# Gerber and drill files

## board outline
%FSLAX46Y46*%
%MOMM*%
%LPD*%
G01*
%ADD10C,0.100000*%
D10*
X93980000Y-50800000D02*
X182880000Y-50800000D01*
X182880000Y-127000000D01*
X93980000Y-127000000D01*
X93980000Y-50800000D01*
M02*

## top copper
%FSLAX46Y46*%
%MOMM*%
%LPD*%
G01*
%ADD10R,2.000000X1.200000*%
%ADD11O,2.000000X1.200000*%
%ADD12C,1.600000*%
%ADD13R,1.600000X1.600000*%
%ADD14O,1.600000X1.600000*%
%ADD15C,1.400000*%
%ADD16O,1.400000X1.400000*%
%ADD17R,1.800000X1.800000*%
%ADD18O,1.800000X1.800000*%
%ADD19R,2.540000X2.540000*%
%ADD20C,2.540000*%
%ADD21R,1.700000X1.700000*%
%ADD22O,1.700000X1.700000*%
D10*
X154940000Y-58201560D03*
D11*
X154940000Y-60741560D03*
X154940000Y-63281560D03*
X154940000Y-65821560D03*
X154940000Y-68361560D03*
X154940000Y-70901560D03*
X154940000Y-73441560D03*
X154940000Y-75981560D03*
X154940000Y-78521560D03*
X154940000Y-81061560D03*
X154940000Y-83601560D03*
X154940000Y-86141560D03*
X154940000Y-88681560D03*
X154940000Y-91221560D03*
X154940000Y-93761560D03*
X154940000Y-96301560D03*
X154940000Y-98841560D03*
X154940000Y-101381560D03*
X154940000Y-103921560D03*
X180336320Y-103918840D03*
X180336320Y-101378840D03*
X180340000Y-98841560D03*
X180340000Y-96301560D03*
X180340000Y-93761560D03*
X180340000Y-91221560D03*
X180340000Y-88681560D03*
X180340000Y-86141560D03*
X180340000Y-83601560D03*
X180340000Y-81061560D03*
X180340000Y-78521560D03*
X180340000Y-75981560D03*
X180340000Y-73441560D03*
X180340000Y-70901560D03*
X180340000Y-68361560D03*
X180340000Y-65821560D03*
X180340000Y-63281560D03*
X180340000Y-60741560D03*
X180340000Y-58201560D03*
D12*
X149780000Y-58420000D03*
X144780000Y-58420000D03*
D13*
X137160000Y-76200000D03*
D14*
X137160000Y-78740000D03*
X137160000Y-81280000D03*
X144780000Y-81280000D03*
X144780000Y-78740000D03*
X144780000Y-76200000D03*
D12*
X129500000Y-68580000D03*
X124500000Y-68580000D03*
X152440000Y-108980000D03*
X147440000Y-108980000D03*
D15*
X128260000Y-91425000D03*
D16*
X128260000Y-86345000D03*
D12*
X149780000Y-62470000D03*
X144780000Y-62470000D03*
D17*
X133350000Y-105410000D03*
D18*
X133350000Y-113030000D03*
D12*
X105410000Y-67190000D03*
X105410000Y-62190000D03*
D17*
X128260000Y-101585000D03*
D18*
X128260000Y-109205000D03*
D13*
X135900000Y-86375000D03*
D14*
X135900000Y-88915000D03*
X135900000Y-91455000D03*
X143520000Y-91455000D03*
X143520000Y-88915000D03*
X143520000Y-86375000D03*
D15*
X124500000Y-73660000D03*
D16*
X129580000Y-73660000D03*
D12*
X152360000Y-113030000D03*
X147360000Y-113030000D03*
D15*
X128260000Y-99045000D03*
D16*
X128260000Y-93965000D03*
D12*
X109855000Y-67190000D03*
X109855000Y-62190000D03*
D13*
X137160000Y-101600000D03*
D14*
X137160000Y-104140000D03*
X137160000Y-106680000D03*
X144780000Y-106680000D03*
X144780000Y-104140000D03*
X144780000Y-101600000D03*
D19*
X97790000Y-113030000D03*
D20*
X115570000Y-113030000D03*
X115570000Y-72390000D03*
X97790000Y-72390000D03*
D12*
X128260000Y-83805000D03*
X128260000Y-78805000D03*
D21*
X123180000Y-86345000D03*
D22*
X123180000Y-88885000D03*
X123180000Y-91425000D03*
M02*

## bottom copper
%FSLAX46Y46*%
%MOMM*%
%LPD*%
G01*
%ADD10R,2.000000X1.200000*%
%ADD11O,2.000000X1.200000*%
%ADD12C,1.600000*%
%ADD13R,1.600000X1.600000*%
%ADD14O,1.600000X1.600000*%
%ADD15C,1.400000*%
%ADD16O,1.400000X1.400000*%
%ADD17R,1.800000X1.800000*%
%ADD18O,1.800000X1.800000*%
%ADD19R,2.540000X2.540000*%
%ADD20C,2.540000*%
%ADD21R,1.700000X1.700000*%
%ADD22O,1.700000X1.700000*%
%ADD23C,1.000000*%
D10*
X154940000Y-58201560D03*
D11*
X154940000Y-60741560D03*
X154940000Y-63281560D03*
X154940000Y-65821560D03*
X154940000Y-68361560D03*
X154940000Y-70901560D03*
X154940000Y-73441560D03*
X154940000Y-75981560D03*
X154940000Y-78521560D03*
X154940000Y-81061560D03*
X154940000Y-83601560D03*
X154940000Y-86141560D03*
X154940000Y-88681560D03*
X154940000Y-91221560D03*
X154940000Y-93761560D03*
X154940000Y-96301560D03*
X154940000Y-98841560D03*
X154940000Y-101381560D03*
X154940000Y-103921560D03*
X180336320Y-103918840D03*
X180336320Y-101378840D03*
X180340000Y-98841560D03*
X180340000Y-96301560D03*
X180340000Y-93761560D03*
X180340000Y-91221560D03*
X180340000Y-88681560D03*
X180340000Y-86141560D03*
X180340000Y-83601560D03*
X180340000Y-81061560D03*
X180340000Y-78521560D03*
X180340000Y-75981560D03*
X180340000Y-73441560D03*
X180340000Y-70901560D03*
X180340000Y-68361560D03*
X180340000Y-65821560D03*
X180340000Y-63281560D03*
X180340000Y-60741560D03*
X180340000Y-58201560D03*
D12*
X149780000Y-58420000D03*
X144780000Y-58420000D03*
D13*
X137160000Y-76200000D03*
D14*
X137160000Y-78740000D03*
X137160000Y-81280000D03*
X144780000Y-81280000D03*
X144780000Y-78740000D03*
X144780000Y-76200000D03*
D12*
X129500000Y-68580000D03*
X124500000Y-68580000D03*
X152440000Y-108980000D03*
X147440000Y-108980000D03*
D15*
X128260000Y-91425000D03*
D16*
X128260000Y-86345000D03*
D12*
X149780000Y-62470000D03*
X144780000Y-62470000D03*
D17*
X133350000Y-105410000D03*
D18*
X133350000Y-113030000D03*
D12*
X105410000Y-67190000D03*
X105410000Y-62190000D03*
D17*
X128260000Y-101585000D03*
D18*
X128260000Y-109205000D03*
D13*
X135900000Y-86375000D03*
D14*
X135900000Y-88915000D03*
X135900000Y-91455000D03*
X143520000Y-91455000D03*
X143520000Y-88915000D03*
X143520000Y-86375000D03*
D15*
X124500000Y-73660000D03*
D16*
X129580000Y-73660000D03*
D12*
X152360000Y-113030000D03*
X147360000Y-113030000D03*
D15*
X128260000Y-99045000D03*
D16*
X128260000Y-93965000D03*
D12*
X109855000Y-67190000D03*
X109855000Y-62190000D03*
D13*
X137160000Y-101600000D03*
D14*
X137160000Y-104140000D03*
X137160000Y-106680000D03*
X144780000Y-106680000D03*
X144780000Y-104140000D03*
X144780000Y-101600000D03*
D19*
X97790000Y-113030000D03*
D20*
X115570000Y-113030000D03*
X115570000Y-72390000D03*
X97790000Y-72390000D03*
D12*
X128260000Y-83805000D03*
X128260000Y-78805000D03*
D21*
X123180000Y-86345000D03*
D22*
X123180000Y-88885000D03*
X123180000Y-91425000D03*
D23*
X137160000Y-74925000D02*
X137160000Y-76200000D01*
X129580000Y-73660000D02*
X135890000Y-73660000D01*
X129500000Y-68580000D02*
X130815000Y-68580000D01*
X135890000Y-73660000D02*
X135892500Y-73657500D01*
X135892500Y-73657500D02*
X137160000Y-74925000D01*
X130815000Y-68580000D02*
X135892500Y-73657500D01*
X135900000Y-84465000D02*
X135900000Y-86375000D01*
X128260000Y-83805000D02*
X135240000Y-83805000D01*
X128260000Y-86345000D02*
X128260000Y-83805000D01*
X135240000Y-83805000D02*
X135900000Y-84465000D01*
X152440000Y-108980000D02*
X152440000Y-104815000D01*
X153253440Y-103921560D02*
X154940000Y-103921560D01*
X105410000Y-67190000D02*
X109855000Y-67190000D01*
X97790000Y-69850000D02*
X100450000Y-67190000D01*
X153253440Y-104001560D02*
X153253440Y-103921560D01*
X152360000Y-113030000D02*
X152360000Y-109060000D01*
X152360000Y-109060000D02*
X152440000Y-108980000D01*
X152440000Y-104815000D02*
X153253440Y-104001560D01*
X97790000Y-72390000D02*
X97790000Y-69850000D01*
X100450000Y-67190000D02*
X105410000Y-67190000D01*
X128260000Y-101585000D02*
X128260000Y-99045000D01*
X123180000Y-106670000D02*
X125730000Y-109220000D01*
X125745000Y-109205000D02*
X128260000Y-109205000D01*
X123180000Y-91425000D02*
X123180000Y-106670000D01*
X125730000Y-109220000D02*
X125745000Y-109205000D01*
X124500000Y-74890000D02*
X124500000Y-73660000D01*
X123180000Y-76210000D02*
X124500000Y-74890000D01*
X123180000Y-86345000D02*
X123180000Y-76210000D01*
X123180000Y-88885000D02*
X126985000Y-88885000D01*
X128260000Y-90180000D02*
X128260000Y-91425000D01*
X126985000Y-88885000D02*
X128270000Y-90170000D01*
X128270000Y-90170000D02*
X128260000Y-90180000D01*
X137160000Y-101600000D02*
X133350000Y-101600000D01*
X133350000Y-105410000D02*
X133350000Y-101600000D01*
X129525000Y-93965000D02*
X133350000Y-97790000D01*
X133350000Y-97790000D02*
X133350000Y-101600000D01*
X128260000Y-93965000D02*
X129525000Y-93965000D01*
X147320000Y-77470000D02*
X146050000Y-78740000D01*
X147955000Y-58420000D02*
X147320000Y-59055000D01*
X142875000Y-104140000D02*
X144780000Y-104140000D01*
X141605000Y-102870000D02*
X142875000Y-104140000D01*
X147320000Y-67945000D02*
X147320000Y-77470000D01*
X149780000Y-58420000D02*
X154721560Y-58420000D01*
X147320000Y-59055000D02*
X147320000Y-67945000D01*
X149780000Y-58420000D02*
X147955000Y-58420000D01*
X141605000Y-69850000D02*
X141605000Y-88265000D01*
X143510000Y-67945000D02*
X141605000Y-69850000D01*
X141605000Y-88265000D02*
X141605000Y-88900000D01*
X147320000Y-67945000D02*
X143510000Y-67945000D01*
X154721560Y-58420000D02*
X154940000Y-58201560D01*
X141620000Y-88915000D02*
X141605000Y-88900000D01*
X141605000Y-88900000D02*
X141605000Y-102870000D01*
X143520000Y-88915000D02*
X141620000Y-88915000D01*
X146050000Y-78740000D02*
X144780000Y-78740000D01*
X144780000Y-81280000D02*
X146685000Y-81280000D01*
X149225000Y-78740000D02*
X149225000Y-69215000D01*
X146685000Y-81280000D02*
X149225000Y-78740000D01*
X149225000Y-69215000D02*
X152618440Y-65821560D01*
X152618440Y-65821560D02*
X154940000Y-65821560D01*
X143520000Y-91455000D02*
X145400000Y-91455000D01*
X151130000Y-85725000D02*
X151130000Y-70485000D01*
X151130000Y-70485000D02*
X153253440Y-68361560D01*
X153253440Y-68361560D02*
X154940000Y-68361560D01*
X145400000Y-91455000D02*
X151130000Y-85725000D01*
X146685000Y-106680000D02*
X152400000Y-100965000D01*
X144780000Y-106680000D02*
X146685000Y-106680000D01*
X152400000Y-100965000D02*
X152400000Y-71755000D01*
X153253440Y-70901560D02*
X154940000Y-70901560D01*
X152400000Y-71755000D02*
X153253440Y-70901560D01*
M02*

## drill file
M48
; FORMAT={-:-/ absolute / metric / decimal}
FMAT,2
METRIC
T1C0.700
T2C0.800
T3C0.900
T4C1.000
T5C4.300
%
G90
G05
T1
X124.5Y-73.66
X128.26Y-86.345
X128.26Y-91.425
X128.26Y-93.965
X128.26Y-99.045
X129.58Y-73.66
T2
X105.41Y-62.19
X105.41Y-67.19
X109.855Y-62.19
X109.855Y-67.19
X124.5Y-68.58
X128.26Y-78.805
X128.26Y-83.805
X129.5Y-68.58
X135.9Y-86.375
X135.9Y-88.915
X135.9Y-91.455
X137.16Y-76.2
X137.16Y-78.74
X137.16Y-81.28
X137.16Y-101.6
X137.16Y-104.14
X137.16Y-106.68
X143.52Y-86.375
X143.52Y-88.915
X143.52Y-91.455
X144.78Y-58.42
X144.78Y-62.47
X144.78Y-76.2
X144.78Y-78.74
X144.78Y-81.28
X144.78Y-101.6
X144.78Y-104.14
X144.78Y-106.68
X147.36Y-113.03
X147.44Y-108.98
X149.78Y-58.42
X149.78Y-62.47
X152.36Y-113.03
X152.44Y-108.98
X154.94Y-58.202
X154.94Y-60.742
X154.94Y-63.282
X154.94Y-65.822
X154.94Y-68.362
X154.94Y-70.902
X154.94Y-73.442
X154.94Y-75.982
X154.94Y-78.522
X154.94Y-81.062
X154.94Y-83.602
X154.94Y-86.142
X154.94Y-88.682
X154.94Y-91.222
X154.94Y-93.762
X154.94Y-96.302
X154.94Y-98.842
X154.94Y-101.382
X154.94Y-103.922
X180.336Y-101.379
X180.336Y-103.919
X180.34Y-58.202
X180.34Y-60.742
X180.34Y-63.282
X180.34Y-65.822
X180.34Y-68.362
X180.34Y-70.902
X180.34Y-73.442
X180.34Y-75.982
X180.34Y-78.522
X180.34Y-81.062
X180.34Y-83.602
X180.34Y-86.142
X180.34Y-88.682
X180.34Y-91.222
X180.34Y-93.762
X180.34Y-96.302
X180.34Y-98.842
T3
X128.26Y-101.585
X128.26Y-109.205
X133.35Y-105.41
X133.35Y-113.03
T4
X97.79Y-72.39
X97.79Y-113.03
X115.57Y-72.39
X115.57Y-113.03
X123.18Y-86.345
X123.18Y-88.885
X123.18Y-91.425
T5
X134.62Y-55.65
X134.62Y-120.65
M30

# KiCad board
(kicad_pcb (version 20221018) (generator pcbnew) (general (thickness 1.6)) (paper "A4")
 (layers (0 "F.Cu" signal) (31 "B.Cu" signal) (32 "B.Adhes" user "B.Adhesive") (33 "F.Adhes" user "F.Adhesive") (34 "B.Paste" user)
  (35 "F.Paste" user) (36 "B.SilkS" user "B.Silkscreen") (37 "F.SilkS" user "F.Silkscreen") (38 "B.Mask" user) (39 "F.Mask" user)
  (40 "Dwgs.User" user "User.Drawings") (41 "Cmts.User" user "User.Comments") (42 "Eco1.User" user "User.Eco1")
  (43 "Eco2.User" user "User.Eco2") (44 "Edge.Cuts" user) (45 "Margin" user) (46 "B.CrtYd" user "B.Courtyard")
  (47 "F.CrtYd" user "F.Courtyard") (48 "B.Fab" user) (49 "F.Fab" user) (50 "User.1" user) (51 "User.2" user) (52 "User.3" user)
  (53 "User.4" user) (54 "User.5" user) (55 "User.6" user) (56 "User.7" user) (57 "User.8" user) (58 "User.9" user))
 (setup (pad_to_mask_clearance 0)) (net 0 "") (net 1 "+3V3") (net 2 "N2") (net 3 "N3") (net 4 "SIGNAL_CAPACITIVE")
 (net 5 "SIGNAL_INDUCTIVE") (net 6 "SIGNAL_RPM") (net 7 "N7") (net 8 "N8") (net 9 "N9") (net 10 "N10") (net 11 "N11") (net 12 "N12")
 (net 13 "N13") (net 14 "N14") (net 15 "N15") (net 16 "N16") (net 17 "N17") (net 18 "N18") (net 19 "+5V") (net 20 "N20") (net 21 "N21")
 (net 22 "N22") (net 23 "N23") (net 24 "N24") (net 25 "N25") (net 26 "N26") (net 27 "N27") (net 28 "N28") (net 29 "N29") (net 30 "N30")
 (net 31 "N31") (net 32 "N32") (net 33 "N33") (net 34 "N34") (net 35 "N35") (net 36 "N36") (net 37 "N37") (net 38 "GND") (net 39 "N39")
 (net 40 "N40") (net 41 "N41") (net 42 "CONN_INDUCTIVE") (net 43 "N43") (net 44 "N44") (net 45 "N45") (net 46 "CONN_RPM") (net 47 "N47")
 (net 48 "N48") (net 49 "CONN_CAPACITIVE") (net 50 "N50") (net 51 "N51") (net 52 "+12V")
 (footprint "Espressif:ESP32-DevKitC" (layer "F.Cu") (at 154.94 58.20156)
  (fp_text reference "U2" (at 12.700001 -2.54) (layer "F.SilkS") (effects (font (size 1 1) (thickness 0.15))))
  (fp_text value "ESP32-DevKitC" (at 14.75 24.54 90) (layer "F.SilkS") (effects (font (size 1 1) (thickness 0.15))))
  (pad "1" thru_hole rect (at 0 0 270) (size 1.2 2) (drill 0.8) (layers "*.Cu" "*.Mask") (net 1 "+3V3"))
  (pad "2" thru_hole oval (at 0 2.54 270) (size 1.2 2) (drill 0.8) (layers "*.Cu" "*.Mask") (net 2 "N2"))
  (pad "3" thru_hole oval (at 0 5.08 270) (size 1.2 2) (drill 0.8) (layers "*.Cu" "*.Mask") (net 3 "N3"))
  (pad "4" thru_hole oval (at 0 7.62 270) (size 1.2 2) (drill 0.8) (layers "*.Cu" "*.Mask") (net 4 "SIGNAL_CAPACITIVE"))
  (pad "5" thru_hole oval (at 0 10.16 270) (size 1.2 2) (drill 0.8) (layers "*.Cu" "*.Mask") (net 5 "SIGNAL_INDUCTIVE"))
  (pad "6" thru_hole oval (at 0 12.7 270) (size 1.2 2) (drill 0.8) (layers "*.Cu" "*.Mask") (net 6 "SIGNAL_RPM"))
  (pad "7" thru_hole oval (at 0 15.24 270) (size 1.2 2) (drill 0.8) (layers "*.Cu" "*.Mask") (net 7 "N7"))
  (pad "8" thru_hole oval (at 0 17.78 270) (size 1.2 2) (drill 0.8) (layers "*.Cu" "*.Mask") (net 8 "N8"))
  (pad "9" thru_hole oval (at 0 20.32 270) (size 1.2 2) (drill 0.8) (layers "*.Cu" "*.Mask") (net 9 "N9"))
  (pad "10" thru_hole oval (at 0 22.86 270) (size 1.2 2) (drill 0.8) (layers "*.Cu" "*.Mask") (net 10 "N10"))
  (pad "11" thru_hole oval (at 0 25.4 270) (size 1.2 2) (drill 0.8) (layers "*.Cu" "*.Mask") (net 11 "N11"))
  (pad "12" thru_hole oval (at 0 27.94 270) (size 1.2 2) (drill 0.8) (layers "*.Cu" "*.Mask") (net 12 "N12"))
  (pad "13" thru_hole oval (at 0 30.48 270) (size 1.2 2) (drill 0.8) (layers "*.Cu" "*.Mask") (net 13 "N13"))
  (pad "14" thru_hole oval (at 0 33.02 270) (size 1.2 2) (drill 0.8) (layers "*.Cu" "*.Mask") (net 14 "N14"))
  (pad "15" thru_hole oval (at 0 35.56 270) (size 1.2 2) (drill 0.8) (layers "*.Cu" "*.Mask") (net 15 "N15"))
  (pad "16" thru_hole oval (at 0 38.1 270) (size 1.2 2) (drill 0.8) (layers "*.Cu" "*.Mask") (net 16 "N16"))
  (pad "17" thru_hole oval (at 0 40.64 270) (size 1.2 2) (drill 0.8) (layers "*.Cu" "*.Mask") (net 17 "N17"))
  (pad "18" thru_hole oval (at 0 43.18 270) (size 1.2 2) (drill 0.8) (layers "*.Cu" "*.Mask") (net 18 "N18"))
  (pad "19" thru_hole oval (at 0 45.72 270) (size 1.2 2) (drill 0.8) (layers "*.Cu" "*.Mask") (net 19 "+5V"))
  (pad "20" thru_hole oval (at 25.39632 45.71728 270) (size 1.2 2) (drill 0.8) (layers "*.Cu" "*.Mask") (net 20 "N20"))
  (pad "21" thru_hole oval (at 25.39632 43.17728 270) (size 1.2 2) (drill 0.8) (layers "*.Cu" "*.Mask") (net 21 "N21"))
  (pad "22" thru_hole oval (at 25.4 40.64 270) (size 1.2 2) (drill 0.8) (layers "*.Cu" "*.Mask") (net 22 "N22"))
  (pad "23" thru_hole oval (at 25.4 38.1 270) (size 1.2 2) (drill 0.8) (layers "*.Cu" "*.Mask") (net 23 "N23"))
  (pad "24" thru_hole oval (at 25.4 35.56 270) (size 1.2 2) (drill 0.8) (layers "*.Cu" "*.Mask") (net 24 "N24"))
  (pad "25" thru_hole oval (at 25.4 33.02 270) (size 1.2 2) (drill 0.8) (layers "*.Cu" "*.Mask") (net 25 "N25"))
  (pad "26" thru_hole oval (at 25.4 30.48 270) (size 1.2 2) (drill 0.8) (layers "*.Cu" "*.Mask") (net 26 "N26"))
  (pad "27" thru_hole oval (at 25.4 27.94 270) (size 1.2 2) (drill 0.8) (layers "*.Cu" "*.Mask") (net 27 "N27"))
  (pad "28" thru_hole oval (at 25.4 25.4 270) (size 1.2 2) (drill 0.8) (layers "*.Cu" "*.Mask") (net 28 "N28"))
  (pad "29" thru_hole oval (at 25.4 22.86 270) (size 1.2 2) (drill 0.8) (layers "*.Cu" "*.Mask") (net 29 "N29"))
  (pad "30" thru_hole oval (at 25.4 20.32 270) (size 1.2 2) (drill 0.8) (layers "*.Cu" "*.Mask") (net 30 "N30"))
  (pad "31" thru_hole oval (at 25.4 17.78 270) (size 1.2 2) (drill 0.8) (layers "*.Cu" "*.Mask") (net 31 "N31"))
  (pad "32" thru_hole oval (at 25.4 15.24 270) (size 1.2 2) (drill 0.8) (layers "*.Cu" "*.Mask") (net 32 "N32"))
  (pad "33" thru_hole oval (at 25.4 12.7 270) (size 1.2 2) (drill 0.8) (layers "*.Cu" "*.Mask") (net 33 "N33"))
  (pad "34" thru_hole oval (at 25.4 10.16 270) (size 1.2 2) (drill 0.8) (layers "*.Cu" "*.Mask") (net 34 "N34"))
  (pad "35" thru_hole oval (at 25.4 7.62 270) (size 1.2 2) (drill 0.8) (layers "*.Cu" "*.Mask") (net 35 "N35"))
  (pad "36" thru_hole oval (at 25.4 5.08 270) (size 1.2 2) (drill 0.8) (layers "*.Cu" "*.Mask") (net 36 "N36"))
  (pad "37" thru_hole oval (at 25.4 2.54 270) (size 1.2 2) (drill 0.8) (layers "*.Cu" "*.Mask") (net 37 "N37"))
  (pad "38" thru_hole oval (at 25.4 0 270) (size 1.2 2) (drill 0.8) (layers "*.Cu" "*.Mask") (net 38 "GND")))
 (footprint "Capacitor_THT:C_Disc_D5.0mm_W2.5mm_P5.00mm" (layer "F.Cu") (at 149.78 58.42 180)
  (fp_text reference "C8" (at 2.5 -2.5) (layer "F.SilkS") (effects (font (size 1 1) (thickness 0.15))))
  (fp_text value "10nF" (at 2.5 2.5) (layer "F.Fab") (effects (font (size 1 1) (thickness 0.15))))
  (pad "1" thru_hole circle (at 0 0 180) (size 1.6 1.6) (drill 0.8) (layers "*.Cu" "*.Mask") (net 1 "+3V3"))
  (pad "2" thru_hole circle (at 5 0 180) (size 1.6 1.6) (drill 0.8) (layers "*.Cu" "*.Mask") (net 38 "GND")))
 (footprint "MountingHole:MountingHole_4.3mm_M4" (layer "F.Cu") (at 134.62 55.65)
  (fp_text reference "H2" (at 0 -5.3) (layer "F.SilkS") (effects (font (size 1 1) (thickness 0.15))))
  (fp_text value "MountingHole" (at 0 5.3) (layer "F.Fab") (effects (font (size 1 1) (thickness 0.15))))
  (pad "" np_thru_hole circle (at 0 0) (size 4.3 4.3) (drill 4.3) (layers "*.Cu" "*.Mask")))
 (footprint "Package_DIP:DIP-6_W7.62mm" (layer "F.Cu") (at 137.16 76.2)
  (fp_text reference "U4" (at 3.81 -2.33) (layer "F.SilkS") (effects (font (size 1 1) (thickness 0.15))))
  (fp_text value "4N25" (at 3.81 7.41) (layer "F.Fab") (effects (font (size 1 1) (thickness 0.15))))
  (pad "1" thru_hole rect (at 0 0) (size 1.6 1.6) (drill 0.8) (layers "*.Cu" "*.Mask") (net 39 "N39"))
  (pad "2" thru_hole oval (at 0 2.54) (size 1.6 1.6) (drill 0.8) (layers "*.Cu" "*.Mask") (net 38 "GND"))
  (pad "3" thru_hole oval (at 0 5.08) (size 1.6 1.6) (drill 0.8) (layers "*.Cu" "*.Mask") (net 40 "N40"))
  (pad "4" thru_hole oval (at 7.62 5.08) (size 1.6 1.6) (drill 0.8) (layers "*.Cu" "*.Mask") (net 4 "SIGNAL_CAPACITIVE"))
  (pad "5" thru_hole oval (at 7.62 2.54) (size 1.6 1.6) (drill 0.8) (layers "*.Cu" "*.Mask") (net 1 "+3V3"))
  (pad "6" thru_hole oval (at 7.62 0) (size 1.6 1.6) (drill 0.8) (layers "*.Cu" "*.Mask") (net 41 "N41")))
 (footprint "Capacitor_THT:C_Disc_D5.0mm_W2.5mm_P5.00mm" (layer "F.Cu") (at 129.5 68.58 180)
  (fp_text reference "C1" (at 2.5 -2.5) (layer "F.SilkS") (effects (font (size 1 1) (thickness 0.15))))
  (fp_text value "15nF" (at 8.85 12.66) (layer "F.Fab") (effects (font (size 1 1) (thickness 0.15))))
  (pad "1" thru_hole circle (at 0 0 180) (size 1.6 1.6) (drill 0.8) (layers "*.Cu" "*.Mask") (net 39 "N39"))
  (pad "2" thru_hole circle (at 5 0 180) (size 1.6 1.6) (drill 0.8) (layers "*.Cu" "*.Mask") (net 38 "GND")))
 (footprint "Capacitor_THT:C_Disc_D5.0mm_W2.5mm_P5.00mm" (layer "F.Cu") (at 152.44 108.98 180)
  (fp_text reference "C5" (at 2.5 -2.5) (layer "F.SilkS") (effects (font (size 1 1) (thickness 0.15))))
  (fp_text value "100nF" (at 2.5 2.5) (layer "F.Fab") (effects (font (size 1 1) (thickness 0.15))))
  (pad "1" thru_hole circle (at 0 0 180) (size 1.6 1.6) (drill 0.8) (layers "*.Cu" "*.Mask") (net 19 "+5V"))
  (pad "2" thru_hole circle (at 5 0 180) (size 1.6 1.6) (drill 0.8) (layers "*.Cu" "*.Mask") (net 38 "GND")))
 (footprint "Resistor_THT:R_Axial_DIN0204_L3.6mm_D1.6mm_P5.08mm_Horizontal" (layer "F.Cu") (at 128.26 91.425 90)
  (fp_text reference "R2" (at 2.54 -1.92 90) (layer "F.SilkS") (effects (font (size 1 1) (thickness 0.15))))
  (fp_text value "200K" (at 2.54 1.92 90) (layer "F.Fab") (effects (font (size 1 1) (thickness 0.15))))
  (pad "1" thru_hole circle (at 0 0 90) (size 1.4 1.4) (drill 0.7) (layers "*.Cu" "*.Mask") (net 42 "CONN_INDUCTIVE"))
  (pad "2" thru_hole oval (at 5.08 0 90) (size 1.4 1.4) (drill 0.7) (layers "*.Cu" "*.Mask") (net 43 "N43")))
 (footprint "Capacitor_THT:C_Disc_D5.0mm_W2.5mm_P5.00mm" (layer "F.Cu") (at 149.78 62.47 180)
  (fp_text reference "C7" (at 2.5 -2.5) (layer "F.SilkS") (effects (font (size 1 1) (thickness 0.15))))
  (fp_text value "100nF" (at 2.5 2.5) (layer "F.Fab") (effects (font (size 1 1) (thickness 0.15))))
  (pad "1" thru_hole circle (at 0 0 180) (size 1.6 1.6) (drill 0.8) (layers "*.Cu" "*.Mask") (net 1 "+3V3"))
  (pad "2" thru_hole circle (at 5 0 180) (size 1.6 1.6) (drill 0.8) (layers "*.Cu" "*.Mask") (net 38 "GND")))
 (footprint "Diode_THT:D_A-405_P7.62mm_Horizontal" (layer "F.Cu") (at 133.35 105.41 -90)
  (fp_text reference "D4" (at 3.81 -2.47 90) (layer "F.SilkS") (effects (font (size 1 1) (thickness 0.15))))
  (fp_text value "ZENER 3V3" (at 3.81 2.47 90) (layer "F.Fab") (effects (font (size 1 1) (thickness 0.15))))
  (pad "1" thru_hole rect (at 0 0 270) (size 1.8 1.8) (drill 0.9) (layers "*.Cu" "*.Mask") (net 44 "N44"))
  (pad "2" thru_hole oval (at 7.62 0 270) (size 1.8 1.8) (drill 0.9) (layers "*.Cu" "*.Mask") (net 38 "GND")))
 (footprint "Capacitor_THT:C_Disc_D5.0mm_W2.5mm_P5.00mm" (layer "F.Cu") (at 105.41 67.19 90)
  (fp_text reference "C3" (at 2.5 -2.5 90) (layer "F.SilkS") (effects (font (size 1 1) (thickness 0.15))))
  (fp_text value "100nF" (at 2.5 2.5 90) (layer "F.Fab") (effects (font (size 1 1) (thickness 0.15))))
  (pad "1" thru_hole circle (at 0 0 90) (size 1.6 1.6) (drill 0.8) (layers "*.Cu" "*.Mask") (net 19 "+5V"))
  (pad "2" thru_hole circle (at 5 0 90) (size 1.6 1.6) (drill 0.8) (layers "*.Cu" "*.Mask") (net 38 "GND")))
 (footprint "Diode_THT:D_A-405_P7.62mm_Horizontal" (layer "F.Cu") (at 128.26 101.585 -90)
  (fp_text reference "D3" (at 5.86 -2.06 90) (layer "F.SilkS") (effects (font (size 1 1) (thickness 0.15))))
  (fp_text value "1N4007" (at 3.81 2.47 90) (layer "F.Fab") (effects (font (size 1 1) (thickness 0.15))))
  (pad "1" thru_hole rect (at 0 0 270) (size 1.8 1.8) (drill 0.9) (layers "*.Cu" "*.Mask") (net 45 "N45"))
  (pad "2" thru_hole oval (at 7.62 0 270) (size 1.8 1.8) (drill 0.9) (layers "*.Cu" "*.Mask") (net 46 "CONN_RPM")))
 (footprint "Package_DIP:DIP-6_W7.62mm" (layer "F.Cu") (at 135.9 86.375)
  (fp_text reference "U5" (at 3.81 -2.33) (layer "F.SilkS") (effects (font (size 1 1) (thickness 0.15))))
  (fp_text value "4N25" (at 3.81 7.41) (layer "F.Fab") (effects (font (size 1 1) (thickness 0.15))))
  (pad "1" thru_hole rect (at 0 0) (size 1.6 1.6) (drill 0.8) (layers "*.Cu" "*.Mask") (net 43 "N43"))
  (pad "2" thru_hole oval (at 0 2.54) (size 1.6 1.6) (drill 0.8) (layers "*.Cu" "*.Mask") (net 38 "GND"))
  (pad "3" thru_hole oval (at 0 5.08) (size 1.6 1.6) (drill 0.8) (layers "*.Cu" "*.Mask") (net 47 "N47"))
  (pad "4" thru_hole oval (at 7.62 5.08) (size 1.6 1.6) (drill 0.8) (layers "*.Cu" "*.Mask") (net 5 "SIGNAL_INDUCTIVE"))
  (pad "5" thru_hole oval (at 7.62 2.54) (size 1.6 1.6) (drill 0.8) (layers "*.Cu" "*.Mask") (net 1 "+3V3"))
  (pad "6" thru_hole oval (at 7.62 0) (size 1.6 1.6) (drill 0.8) (layers "*.Cu" "*.Mask") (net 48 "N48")))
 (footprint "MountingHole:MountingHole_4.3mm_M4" (layer "F.Cu") (at 134.62 120.65)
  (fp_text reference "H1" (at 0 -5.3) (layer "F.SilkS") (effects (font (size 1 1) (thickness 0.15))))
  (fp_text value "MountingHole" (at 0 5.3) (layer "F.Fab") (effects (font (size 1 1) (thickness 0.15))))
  (pad "" np_thru_hole circle (at 0 0) (size 4.3 4.3) (drill 4.3) (layers "*.Cu" "*.Mask")))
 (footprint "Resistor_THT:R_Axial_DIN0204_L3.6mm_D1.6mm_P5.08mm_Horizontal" (layer "F.Cu") (at 124.5 73.66)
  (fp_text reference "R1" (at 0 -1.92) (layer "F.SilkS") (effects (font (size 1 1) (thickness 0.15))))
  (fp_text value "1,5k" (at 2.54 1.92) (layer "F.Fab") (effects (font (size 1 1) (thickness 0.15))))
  (pad "1" thru_hole circle (at 0 0) (size 1.4 1.4) (drill 0.7) (layers "*.Cu" "*.Mask") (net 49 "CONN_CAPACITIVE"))
  (pad "2" thru_hole oval (at 5.08 0) (size 1.4 1.4) (drill 0.7) (layers "*.Cu" "*.Mask") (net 39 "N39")))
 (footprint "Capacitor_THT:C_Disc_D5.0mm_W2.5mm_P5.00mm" (layer "F.Cu") (at 152.36 113.03 180)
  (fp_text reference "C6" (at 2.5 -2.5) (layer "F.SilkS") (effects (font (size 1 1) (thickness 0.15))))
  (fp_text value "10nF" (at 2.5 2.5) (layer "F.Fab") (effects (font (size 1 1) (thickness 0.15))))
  (pad "1" thru_hole circle (at 0 0 180) (size 1.6 1.6) (drill 0.8) (layers "*.Cu" "*.Mask") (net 19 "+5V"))
  (pad "2" thru_hole circle (at 5 0 180) (size 1.6 1.6) (drill 0.8) (layers "*.Cu" "*.Mask") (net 38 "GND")))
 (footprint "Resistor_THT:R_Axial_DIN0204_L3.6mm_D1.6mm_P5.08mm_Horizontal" (layer "F.Cu") (at 128.26 99.045 90)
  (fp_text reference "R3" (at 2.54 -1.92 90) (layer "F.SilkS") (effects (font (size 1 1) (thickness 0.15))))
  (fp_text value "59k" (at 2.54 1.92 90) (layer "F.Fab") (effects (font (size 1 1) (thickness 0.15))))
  (pad "1" thru_hole circle (at 0 0 90) (size 1.4 1.4) (drill 0.7) (layers "*.Cu" "*.Mask") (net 45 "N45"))
  (pad "2" thru_hole oval (at 5.08 0 90) (size 1.4 1.4) (drill 0.7) (layers "*.Cu" "*.Mask") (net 44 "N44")))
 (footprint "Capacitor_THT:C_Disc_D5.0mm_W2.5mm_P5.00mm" (layer "F.Cu") (at 109.855 67.19 90)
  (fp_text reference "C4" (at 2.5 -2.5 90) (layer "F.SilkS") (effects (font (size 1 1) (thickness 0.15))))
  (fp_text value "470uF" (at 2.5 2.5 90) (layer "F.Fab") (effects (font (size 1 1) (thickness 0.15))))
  (pad "1" thru_hole circle (at 0 0 90) (size 1.6 1.6) (drill 0.8) (layers "*.Cu" "*.Mask") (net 19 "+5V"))
  (pad "2" thru_hole circle (at 5 0 90) (size 1.6 1.6) (drill 0.8) (layers "*.Cu" "*.Mask") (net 38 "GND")))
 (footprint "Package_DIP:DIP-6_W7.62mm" (layer "F.Cu") (at 137.16 101.6)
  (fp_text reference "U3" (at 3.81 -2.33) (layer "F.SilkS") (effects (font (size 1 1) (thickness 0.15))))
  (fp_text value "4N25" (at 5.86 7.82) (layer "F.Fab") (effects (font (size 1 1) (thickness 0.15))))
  (pad "1" thru_hole rect (at 0 0) (size 1.6 1.6) (drill 0.8) (layers "*.Cu" "*.Mask") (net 44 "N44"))
  (pad "2" thru_hole oval (at 0 2.54) (size 1.6 1.6) (drill 0.8) (layers "*.Cu" "*.Mask") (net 38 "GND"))
  (pad "3" thru_hole oval (at 0 5.08) (size 1.6 1.6) (drill 0.8) (layers "*.Cu" "*.Mask") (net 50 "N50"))
  (pad "4" thru_hole oval (at 7.62 5.08) (size 1.6 1.6) (drill 0.8) (layers "*.Cu" "*.Mask") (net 6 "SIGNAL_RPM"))
  (pad "5" thru_hole oval (at 7.62 2.54) (size 1.6 1.6) (drill 0.8) (layers "*.Cu" "*.Mask") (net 1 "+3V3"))
  (pad "6" thru_hole oval (at 7.62 0) (size 1.6 1.6) (drill 0.8) (layers "*.Cu" "*.Mask") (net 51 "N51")))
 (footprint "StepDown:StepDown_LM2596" (layer "F.Cu") (at 97.79 113.03 90)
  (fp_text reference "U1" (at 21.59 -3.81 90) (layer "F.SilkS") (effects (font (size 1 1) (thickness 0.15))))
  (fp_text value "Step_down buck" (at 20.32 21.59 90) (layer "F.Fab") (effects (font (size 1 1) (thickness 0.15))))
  (pad "1" thru_hole rect (at 0 0 90) (size 2.54 2.54) (drill 1) (layers "*.Cu" "*.Mask") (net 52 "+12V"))
  (pad "2" thru_hole circle (at 0 17.78 90) (size 2.54 2.54) (drill 1) (layers "*.Cu" "*.Mask") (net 38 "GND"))
  (pad "3" thru_hole circle (at 40.64 17.78 90) (size 2.54 2.54) (drill 1) (layers "*.Cu" "*.Mask") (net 38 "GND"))
  (pad "4" thru_hole circle (at 40.64 0 90) (size 2.54 2.54) (drill 1) (layers "*.Cu" "*.Mask") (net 19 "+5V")))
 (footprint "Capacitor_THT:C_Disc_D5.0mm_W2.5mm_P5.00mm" (layer "F.Cu") (at 128.26 83.805 90)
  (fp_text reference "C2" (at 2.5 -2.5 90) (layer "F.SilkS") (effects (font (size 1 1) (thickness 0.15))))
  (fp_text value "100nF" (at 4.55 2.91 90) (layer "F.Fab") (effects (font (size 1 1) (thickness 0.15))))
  (pad "1" thru_hole circle (at 0 0 90) (size 1.6 1.6) (drill 0.8) (layers "*.Cu" "*.Mask") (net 43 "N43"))
  (pad "2" thru_hole circle (at 5 0 90) (size 1.6 1.6) (drill 0.8) (layers "*.Cu" "*.Mask") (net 38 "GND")))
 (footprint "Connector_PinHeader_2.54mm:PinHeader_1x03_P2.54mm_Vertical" (layer "F.Cu") (at 123.18 86.345)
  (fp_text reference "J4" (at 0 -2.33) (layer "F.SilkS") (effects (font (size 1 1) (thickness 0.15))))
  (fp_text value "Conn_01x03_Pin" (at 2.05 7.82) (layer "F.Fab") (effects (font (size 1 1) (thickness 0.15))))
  (pad "1" thru_hole rect (at 0 0) (size 1.7 1.7) (drill 1) (layers "*.Cu" "*.Mask") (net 49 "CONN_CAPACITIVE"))
  (pad "2" thru_hole oval (at 0 2.54) (size 1.7 1.7) (drill 1) (layers "*.Cu" "*.Mask") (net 42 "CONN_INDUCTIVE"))
  (pad "3" thru_hole oval (at 0 5.08) (size 1.7 1.7) (drill 1) (layers "*.Cu" "*.Mask") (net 46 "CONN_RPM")))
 (gr_rect (start 93.98 50.8) (end 182.88 127) (stroke (width 0.1) (type default)) (fill none) (layer "Edge.Cuts"))
 (segment (start 137.16 74.925) (end 137.16 76.2) (width 1) (layer "B.Cu") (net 39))
 (segment (start 129.58 73.66) (end 135.89 73.66) (width 1) (layer "B.Cu") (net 39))
 (segment (start 129.5 68.58) (end 130.815 68.58) (width 1) (layer "B.Cu") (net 39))
 (segment (start 135.89 73.66) (end 135.8925 73.6575) (width 1) (layer "B.Cu") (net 39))
 (segment (start 135.8925 73.6575) (end 137.16 74.925) (width 1) (layer "B.Cu") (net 39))
 (segment (start 130.815 68.58) (end 135.8925 73.6575) (width 1) (layer "B.Cu") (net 39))
 (segment (start 135.9 84.465) (end 135.9 86.375) (width 1) (layer "B.Cu") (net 43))
 (segment (start 128.26 83.805) (end 135.24 83.805) (width 1) (layer "B.Cu") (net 43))
 (segment (start 128.26 86.345) (end 128.26 83.805) (width 1) (layer "B.Cu") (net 43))
 (segment (start 135.24 83.805) (end 135.9 84.465) (width 1) (layer "B.Cu") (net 43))
 (segment (start 152.44 108.98) (end 152.44 104.815) (width 1) (layer "B.Cu") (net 19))
 (segment (start 153.25344 103.92156) (end 154.94 103.92156) (width 1) (layer "B.Cu") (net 19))
 (segment (start 105.41 67.19) (end 109.855 67.19) (width 1) (layer "B.Cu") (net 19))
 (segment (start 97.79 69.85) (end 100.45 67.19) (width 1) (layer "B.Cu") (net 19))
 (segment (start 153.25344 104.00156) (end 153.25344 103.92156) (width 1) (layer "B.Cu") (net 19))
 (segment (start 152.36 113.03) (end 152.36 109.06) (width 1) (layer "B.Cu") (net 19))
 (segment (start 152.36 109.06) (end 152.44 108.98) (width 1) (layer "B.Cu") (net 19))
 (segment (start 152.44 104.815) (end 153.25344 104.00156) (width 1) (layer "B.Cu") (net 19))
 (segment (start 97.79 72.39) (end 97.79 69.85) (width 1) (layer "B.Cu") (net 19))
 (segment (start 100.45 67.19) (end 105.41 67.19) (width 1) (layer "B.Cu") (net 19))
 (segment (start 128.26 101.585) (end 128.26 99.045) (width 1) (layer "B.Cu") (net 45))
 (segment (start 123.18 106.67) (end 125.73 109.22) (width 1) (layer "B.Cu") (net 46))
 (segment (start 125.745 109.205) (end 128.26 109.205) (width 1) (layer "B.Cu") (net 46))
 (segment (start 123.18 91.425) (end 123.18 106.67) (width 1) (layer "B.Cu") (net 46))
 (segment (start 125.73 109.22) (end 125.745 109.205) (width 1) (layer "B.Cu") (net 46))
 (segment (start 124.5 74.89) (end 124.5 73.66) (width 1) (layer "B.Cu") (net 49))
 (segment (start 123.18 76.21) (end 124.5 74.89) (width 1) (layer "B.Cu") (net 49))
 (segment (start 123.18 86.345) (end 123.18 76.21) (width 1) (layer "B.Cu") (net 49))
 (segment (start 123.18 88.885) (end 126.985 88.885) (width 1) (layer "B.Cu") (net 42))
 (segment (start 128.26 90.18) (end 128.26 91.425) (width 1) (layer "B.Cu") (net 42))
 (segment (start 126.985 88.885) (end 128.27 90.17) (width 1) (layer "B.Cu") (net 42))
 (segment (start 128.27 90.17) (end 128.26 90.18) (width 1) (layer "B.Cu") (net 42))
 (segment (start 137.16 101.6) (end 133.35 101.6) (width 1) (layer "B.Cu") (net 44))
 (segment (start 133.35 105.41) (end 133.35 101.6) (width 1) (layer "B.Cu") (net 44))
 (segment (start 129.525 93.965) (end 133.35 97.79) (width 1) (layer "B.Cu") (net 44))
 (segment (start 133.35 97.79) (end 133.35 101.6) (width 1) (layer "B.Cu") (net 44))
 (segment (start 128.26 93.965) (end 129.525 93.965) (width 1) (layer "B.Cu") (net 44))
 (segment (start 147.32 77.47) (end 146.05 78.74) (width 1) (layer "B.Cu") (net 1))
 (segment (start 147.955 58.42) (end 147.32 59.055) (width 1) (layer "B.Cu") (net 1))
 (segment (start 142.875 104.14) (end 144.78 104.14) (width 1) (layer "B.Cu") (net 1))
 (segment (start 141.605 102.87) (end 142.875 104.14) (width 1) (layer "B.Cu") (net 1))
 (segment (start 147.32 67.945) (end 147.32 77.47) (width 1) (layer "B.Cu") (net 1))
 (segment (start 149.78 58.42) (end 154.72156 58.42) (width 1) (layer "B.Cu") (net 1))
 (segment (start 147.32 59.055) (end 147.32 67.945) (width 1) (layer "B.Cu") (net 1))
 (segment (start 149.78 58.42) (end 147.955 58.42) (width 1) (layer "B.Cu") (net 1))
 (segment (start 141.605 69.85) (end 141.605 88.265) (width 1) (layer "B.Cu") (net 1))
 (segment (start 143.51 67.945) (end 141.605 69.85) (width 1) (layer "B.Cu") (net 1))
 (segment (start 141.605 88.265) (end 141.605 88.9) (width 1) (layer "B.Cu") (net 1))
 (segment (start 147.32 67.945) (end 143.51 67.945) (width 1) (layer "B.Cu") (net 1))
 (segment (start 154.72156 58.42) (end 154.94 58.20156) (width 1) (layer "B.Cu") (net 1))
 (segment (start 141.62 88.915) (end 141.605 88.9) (width 1) (layer "B.Cu") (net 1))
 (segment (start 141.605 88.9) (end 141.605 102.87) (width 1) (layer "B.Cu") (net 1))
 (segment (start 143.52 88.915) (end 141.62 88.915) (width 1) (layer "B.Cu") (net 1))
 (segment (start 146.05 78.74) (end 144.78 78.74) (width 1) (layer "B.Cu") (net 1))
 (segment (start 144.78 81.28) (end 146.685 81.28) (width 1) (layer "B.Cu") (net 4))
 (segment (start 149.225 78.74) (end 149.225 69.215) (width 1) (layer "B.Cu") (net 4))
 (segment (start 146.685 81.28) (end 149.225 78.74) (width 1) (layer "B.Cu") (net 4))
 (segment (start 149.225 69.215) (end 152.61844 65.82156) (width 1) (layer "B.Cu") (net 4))
 (segment (start 152.61844 65.82156) (end 154.94 65.82156) (width 1) (layer "B.Cu") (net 4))
 (segment (start 143.52 91.455) (end 145.4 91.455) (width 1) (layer "B.Cu") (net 5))
 (segment (start 151.13 85.725) (end 151.13 70.485) (width 1) (layer "B.Cu") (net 5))
 (segment (start 151.13 70.485) (end 153.25344 68.36156) (width 1) (layer "B.Cu") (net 5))
 (segment (start 153.25344 68.36156) (end 154.94 68.36156) (width 1) (layer "B.Cu") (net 5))
 (segment (start 145.4 91.455) (end 151.13 85.725) (width 1) (layer "B.Cu") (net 5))
 (segment (start 146.685 106.68) (end 152.4 100.965) (width 1) (layer "B.Cu") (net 6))
 (segment (start 144.78 106.68) (end 146.685 106.68) (width 1) (layer "B.Cu") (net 6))
 (segment (start 152.4 100.965) (end 152.4 71.755) (width 1) (layer "B.Cu") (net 6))
 (segment (start 153.25344 70.90156) (end 154.94 70.90156) (width 1) (layer "B.Cu") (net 6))
 (segment (start 152.4 71.755) (end 153.25344 70.90156) (width 1) (layer "B.Cu") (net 6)))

